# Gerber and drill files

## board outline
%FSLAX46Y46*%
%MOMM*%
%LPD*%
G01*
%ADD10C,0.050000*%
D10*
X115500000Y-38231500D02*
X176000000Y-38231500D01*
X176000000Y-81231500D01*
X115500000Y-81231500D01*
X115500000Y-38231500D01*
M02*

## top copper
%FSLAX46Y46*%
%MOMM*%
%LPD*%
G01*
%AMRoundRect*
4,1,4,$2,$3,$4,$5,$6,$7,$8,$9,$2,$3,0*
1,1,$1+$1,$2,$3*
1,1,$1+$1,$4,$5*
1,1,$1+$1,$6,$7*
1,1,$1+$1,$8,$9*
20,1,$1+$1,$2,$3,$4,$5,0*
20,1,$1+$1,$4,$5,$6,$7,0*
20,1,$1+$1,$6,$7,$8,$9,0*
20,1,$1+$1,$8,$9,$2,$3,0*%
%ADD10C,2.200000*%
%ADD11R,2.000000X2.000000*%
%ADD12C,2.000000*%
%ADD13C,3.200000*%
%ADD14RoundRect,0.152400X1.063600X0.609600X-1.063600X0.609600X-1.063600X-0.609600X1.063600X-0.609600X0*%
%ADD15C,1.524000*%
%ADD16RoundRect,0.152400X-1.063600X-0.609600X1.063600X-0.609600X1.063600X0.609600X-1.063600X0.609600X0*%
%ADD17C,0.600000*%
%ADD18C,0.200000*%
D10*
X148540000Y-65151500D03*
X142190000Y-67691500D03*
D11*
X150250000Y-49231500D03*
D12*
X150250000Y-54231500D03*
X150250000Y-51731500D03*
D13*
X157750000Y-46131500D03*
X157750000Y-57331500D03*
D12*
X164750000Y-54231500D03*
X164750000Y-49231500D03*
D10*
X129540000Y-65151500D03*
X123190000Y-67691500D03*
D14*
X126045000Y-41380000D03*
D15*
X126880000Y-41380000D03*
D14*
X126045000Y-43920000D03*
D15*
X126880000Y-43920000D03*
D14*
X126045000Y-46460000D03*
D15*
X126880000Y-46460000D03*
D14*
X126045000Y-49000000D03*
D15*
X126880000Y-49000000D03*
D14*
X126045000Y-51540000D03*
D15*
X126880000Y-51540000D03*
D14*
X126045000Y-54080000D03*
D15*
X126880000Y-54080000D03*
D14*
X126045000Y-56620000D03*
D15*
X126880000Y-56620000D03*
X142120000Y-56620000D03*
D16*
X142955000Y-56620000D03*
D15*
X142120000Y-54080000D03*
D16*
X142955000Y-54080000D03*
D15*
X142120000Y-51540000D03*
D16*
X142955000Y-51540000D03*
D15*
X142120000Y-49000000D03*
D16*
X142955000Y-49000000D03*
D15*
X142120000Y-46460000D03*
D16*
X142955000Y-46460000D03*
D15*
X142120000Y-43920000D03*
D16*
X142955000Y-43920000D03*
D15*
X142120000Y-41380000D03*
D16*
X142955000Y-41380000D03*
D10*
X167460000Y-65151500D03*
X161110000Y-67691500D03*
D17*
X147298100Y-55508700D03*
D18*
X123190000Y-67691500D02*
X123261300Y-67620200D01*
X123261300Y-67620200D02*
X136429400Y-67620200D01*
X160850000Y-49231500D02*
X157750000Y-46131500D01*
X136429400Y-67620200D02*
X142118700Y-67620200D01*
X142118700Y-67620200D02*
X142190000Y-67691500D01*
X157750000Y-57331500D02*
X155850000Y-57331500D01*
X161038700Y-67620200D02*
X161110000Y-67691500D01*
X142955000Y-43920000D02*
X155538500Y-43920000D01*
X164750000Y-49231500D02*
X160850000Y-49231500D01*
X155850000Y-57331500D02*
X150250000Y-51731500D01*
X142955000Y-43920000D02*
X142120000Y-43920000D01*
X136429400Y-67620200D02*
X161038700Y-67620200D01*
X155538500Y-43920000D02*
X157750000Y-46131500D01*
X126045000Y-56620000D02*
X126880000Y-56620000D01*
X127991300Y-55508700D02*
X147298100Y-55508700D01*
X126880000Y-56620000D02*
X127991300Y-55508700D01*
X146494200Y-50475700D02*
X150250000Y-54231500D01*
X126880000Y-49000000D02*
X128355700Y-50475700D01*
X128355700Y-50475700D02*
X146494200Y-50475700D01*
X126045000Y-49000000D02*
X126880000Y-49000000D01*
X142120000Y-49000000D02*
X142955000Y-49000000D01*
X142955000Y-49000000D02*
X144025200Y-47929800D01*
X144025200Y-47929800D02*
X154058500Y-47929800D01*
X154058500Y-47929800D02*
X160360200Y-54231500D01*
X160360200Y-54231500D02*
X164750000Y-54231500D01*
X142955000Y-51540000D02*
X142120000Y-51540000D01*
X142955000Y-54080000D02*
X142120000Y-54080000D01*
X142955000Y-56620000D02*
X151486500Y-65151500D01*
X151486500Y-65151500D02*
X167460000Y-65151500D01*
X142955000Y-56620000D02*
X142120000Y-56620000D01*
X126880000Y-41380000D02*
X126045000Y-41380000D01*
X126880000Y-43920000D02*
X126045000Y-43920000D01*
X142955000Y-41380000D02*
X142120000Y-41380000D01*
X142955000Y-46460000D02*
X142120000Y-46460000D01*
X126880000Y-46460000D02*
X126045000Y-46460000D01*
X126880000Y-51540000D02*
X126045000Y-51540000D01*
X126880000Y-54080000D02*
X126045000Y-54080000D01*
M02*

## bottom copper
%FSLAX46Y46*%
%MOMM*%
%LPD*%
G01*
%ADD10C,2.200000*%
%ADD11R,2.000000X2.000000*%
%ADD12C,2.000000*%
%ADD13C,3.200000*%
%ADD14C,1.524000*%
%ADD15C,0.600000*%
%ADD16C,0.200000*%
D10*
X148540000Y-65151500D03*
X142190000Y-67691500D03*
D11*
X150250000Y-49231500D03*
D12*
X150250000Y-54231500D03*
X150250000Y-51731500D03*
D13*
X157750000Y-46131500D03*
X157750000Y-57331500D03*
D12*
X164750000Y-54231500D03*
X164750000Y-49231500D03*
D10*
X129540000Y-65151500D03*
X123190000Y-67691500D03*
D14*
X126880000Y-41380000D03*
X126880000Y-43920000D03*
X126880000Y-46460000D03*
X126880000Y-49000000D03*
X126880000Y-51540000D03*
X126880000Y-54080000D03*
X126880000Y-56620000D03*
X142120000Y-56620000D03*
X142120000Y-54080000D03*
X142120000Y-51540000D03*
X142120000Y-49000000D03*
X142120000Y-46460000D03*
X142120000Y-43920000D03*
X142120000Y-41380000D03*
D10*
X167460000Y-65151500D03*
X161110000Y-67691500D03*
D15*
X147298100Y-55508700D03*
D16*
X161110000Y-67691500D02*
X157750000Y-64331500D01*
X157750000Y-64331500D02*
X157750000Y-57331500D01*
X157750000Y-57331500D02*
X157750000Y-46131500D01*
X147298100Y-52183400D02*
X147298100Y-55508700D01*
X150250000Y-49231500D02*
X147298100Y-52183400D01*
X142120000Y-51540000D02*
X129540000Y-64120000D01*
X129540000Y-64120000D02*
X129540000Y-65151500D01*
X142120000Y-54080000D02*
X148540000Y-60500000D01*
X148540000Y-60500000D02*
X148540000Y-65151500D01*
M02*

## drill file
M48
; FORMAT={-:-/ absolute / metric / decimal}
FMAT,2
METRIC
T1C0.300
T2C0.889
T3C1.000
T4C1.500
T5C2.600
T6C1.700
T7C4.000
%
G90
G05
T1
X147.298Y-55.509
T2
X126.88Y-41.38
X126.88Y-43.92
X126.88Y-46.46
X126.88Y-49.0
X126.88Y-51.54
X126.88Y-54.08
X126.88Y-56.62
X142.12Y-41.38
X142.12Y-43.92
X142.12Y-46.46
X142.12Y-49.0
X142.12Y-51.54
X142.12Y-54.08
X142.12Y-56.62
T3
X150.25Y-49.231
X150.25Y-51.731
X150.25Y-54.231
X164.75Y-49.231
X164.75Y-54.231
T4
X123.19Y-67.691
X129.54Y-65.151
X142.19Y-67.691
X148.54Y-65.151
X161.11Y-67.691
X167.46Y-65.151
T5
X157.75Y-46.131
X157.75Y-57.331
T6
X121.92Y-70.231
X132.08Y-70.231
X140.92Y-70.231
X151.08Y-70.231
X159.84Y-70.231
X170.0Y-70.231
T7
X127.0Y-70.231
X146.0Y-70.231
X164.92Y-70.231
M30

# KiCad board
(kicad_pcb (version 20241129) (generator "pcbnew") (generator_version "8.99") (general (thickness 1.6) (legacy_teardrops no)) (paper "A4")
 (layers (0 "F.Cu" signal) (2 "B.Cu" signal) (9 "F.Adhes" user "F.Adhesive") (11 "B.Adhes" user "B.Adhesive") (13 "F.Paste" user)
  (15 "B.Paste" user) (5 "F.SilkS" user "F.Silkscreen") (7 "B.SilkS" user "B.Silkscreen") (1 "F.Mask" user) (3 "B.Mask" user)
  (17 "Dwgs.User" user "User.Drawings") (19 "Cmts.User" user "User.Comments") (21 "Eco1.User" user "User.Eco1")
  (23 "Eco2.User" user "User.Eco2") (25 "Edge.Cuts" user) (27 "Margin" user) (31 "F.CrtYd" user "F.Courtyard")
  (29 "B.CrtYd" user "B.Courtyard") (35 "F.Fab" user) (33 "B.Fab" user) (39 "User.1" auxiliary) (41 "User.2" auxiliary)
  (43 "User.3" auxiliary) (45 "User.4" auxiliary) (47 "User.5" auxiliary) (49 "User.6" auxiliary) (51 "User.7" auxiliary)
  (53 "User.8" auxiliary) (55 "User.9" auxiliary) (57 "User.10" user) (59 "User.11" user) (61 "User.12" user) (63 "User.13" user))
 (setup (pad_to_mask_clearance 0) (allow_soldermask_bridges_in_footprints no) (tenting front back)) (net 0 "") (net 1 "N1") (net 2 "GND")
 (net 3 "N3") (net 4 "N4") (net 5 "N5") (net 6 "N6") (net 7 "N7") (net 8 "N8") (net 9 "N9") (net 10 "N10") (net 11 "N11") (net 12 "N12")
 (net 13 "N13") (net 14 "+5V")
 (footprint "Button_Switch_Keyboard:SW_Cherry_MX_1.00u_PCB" (layer "F.Cu") (at 148.54 65.1515)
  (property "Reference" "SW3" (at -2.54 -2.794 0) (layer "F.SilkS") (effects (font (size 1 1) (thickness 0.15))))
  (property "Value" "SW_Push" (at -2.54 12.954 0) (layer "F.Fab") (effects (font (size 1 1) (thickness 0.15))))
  (pad "" np_thru_hole circle (at -7.62 5.08) (size 1.7 1.7) (drill 1.7) (layers "*.Cu" "*.Mask"))
  (pad "" np_thru_hole circle (at -2.54 5.08) (size 4 4) (drill 4) (layers "*.Cu" "*.Mask"))
  (pad "" np_thru_hole circle (at 2.54 5.08) (size 1.7 1.7) (drill 1.7) (layers "*.Cu" "*.Mask"))
  (pad "1" thru_hole circle (at 0 0) (size 2.2 2.2) (drill 1.5) (layers "*.Cu" "*.Mask") (remove_unused_layers no) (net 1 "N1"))
  (pad "2" thru_hole circle (at -6.35 2.54) (size 2.2 2.2) (drill 1.5) (layers "*.Cu" "*.Mask") (remove_unused_layers no) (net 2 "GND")))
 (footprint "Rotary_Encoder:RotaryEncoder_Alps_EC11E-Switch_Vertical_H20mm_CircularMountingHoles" (layer "F.Cu") (at 150.25 49.2315)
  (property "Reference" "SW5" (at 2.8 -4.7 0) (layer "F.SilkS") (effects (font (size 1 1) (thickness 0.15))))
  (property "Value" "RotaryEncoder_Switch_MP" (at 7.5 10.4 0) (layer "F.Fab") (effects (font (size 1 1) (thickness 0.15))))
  (pad "A" thru_hole rect (at 0 0) (size 2 2) (drill 1) (layers "*.Cu" "*.Mask") (remove_unused_layers no) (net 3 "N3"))
  (pad "B" thru_hole circle (at 0 5) (size 2 2) (drill 1) (layers "*.Cu" "*.Mask") (remove_unused_layers no) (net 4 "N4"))
  (pad "C" thru_hole circle (at 0 2.5) (size 2 2) (drill 1) (layers "*.Cu" "*.Mask") (remove_unused_layers no) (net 2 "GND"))
  (pad "MP" thru_hole circle (at 7.5 -3.1) (size 3.2 3.2) (drill 2.6) (layers "*.Cu" "*.Mask") (remove_unused_layers no) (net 2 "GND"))
  (pad "MP" thru_hole circle (at 7.5 8.1) (size 3.2 3.2) (drill 2.6) (layers "*.Cu" "*.Mask") (remove_unused_layers no) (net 2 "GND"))
  (pad "S1" thru_hole circle (at 14.5 5) (size 2 2) (drill 1) (layers "*.Cu" "*.Mask") (remove_unused_layers no) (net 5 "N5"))
  (pad "S2" thru_hole circle (at 14.5 0) (size 2 2) (drill 1) (layers "*.Cu" "*.Mask") (remove_unused_layers no) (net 2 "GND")))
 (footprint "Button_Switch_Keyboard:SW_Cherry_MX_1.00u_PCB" (layer "F.Cu") (at 129.54 65.1515)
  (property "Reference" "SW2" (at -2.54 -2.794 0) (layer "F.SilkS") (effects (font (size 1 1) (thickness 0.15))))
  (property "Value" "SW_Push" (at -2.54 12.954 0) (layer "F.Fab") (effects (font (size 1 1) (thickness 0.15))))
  (pad "" np_thru_hole circle (at -7.62 5.08) (size 1.7 1.7) (drill 1.7) (layers "*.Cu" "*.Mask"))
  (pad "" np_thru_hole circle (at -2.54 5.08) (size 4 4) (drill 4) (layers "*.Cu" "*.Mask"))
  (pad "" np_thru_hole circle (at 2.54 5.08) (size 1.7 1.7) (drill 1.7) (layers "*.Cu" "*.Mask"))
  (pad "1" thru_hole circle (at 0 0) (size 2.2 2.2) (drill 1.5) (layers "*.Cu" "*.Mask") (remove_unused_layers no) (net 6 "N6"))
  (pad "2" thru_hole circle (at -6.35 2.54) (size 2.2 2.2) (drill 1.5) (layers "*.Cu" "*.Mask") (remove_unused_layers no) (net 2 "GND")))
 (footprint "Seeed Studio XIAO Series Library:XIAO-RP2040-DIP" (layer "F.Cu") (at 134.5 49)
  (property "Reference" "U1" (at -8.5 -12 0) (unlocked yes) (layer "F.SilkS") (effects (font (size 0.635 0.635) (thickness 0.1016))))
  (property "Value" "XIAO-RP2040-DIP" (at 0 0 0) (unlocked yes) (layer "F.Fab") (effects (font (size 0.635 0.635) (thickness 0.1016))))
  (pad "1" smd roundrect (at -8.455 -7.62 180) (size 2.432 1.524) (layers "F.Cu" "F.Mask") (roundrect_rratio 0.1) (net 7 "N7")
   (thermal_bridge_angle 45))
  (pad "1" thru_hole circle (at -7.62 -7.62 180) (size 1.524 1.524) (drill 0.889) (layers "*.Cu" "*.Mask") (remove_unused_layers no)
   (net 7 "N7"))
  (pad "2" smd roundrect (at -8.455 -5.08 180) (size 2.432 1.524) (layers "F.Cu" "F.Mask") (roundrect_rratio 0.1) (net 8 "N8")
   (thermal_bridge_angle 45))
  (pad "2" thru_hole circle (at -7.62 -5.08 180) (size 1.524 1.524) (drill 0.889) (layers "*.Cu" "*.Mask") (remove_unused_layers no)
   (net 8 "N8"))
  (pad "3" smd roundrect (at -8.455 -2.54 180) (size 2.432 1.524) (layers "F.Cu" "F.Mask") (roundrect_rratio 0.1) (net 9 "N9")
   (thermal_bridge_angle 45))
  (pad "3" thru_hole circle (at -7.62 -2.54 180) (size 1.524 1.524) (drill 0.889) (layers "*.Cu" "*.Mask") (remove_unused_layers no)
   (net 9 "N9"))
  (pad "4" smd roundrect (at -8.455 0 180) (size 2.432 1.524) (layers "F.Cu" "F.Mask") (roundrect_rratio 0.1) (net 4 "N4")
   (thermal_bridge_angle 45))
  (pad "4" thru_hole circle (at -7.62 0 180) (size 1.524 1.524) (drill 0.889) (layers "*.Cu" "*.Mask") (remove_unused_layers no)
   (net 4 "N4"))
  (pad "5" smd roundrect (at -8.455 2.54 180) (size 2.432 1.524) (layers "F.Cu" "F.Mask") (roundrect_rratio 0.1) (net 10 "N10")
   (thermal_bridge_angle 45))
  (pad "5" thru_hole circle (at -7.62 2.54 180) (size 1.524 1.524) (drill 0.889) (layers "*.Cu" "*.Mask") (remove_unused_layers no)
   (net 10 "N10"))
  (pad "6" smd roundrect (at -8.455 5.08 180) (size 2.432 1.524) (layers "F.Cu" "F.Mask") (roundrect_rratio 0.1) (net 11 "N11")
   (thermal_bridge_angle 45))
  (pad "6" thru_hole circle (at -7.62 5.08 180) (size 1.524 1.524) (drill 0.889) (layers "*.Cu" "*.Mask") (remove_unused_layers no)
   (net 11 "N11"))
  (pad "7" smd roundrect (at -8.455 7.62 180) (size 2.432 1.524) (layers "F.Cu" "F.Mask") (roundrect_rratio 0.1) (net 3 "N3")
   (thermal_bridge_angle 45))
  (pad "7" thru_hole circle (at -7.62 7.62 180) (size 1.524 1.524) (drill 0.889) (layers "*.Cu" "*.Mask") (remove_unused_layers no)
   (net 3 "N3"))
  (pad "8" thru_hole circle (at 7.62 7.62) (size 1.524 1.524) (drill 0.889) (layers "*.Cu" "*.Mask") (remove_unused_layers no)
   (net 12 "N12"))
  (pad "8" smd roundrect (at 8.455 7.62) (size 2.432 1.524) (layers "F.Cu" "F.Mask") (roundrect_rratio 0.1) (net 12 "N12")
   (thermal_bridge_angle 45))
  (pad "9" thru_hole circle (at 7.62 5.08) (size 1.524 1.524) (drill 0.889) (layers "*.Cu" "*.Mask") (remove_unused_layers no) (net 1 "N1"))
  (pad "9" smd roundrect (at 8.455 5.08) (size 2.432 1.524) (layers "F.Cu" "F.Mask") (roundrect_rratio 0.1) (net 1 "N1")
   (thermal_bridge_angle 45))
  (pad "10" thru_hole circle (at 7.62 2.54) (size 1.524 1.524) (drill 0.889) (layers "*.Cu" "*.Mask") (remove_unused_layers no) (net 6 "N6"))
  (pad "10" smd roundrect (at 8.455 2.54) (size 2.432 1.524) (layers "F.Cu" "F.Mask") (roundrect_rratio 0.1) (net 6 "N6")
   (thermal_bridge_angle 45))
  (pad "11" thru_hole circle (at 7.62 0) (size 1.524 1.524) (drill 0.889) (layers "*.Cu" "*.Mask") (remove_unused_layers no) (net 5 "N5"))
  (pad "11" smd roundrect (at 8.455 0) (size 2.432 1.524) (layers "F.Cu" "F.Mask") (roundrect_rratio 0.1) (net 5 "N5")
   (thermal_bridge_angle 45))
  (pad "12" thru_hole circle (at 7.62 -2.54) (size 1.524 1.524) (drill 0.889) (layers "*.Cu" "*.Mask") (remove_unused_layers no)
   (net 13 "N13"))
  (pad "12" smd roundrect (at 8.455 -2.54) (size 2.432 1.524) (layers "F.Cu" "F.Mask") (roundrect_rratio 0.1) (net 13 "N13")
   (thermal_bridge_angle 45))
  (pad "13" thru_hole circle (at 7.62 -5.08) (size 1.524 1.524) (drill 0.889) (layers "*.Cu" "*.Mask") (remove_unused_layers no)
   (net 2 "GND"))
  (pad "13" smd roundrect (at 8.455 -5.08) (size 2.432 1.524) (layers "F.Cu" "F.Mask") (roundrect_rratio 0.1) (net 2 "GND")
   (thermal_bridge_angle 45))
  (pad "14" thru_hole circle (at 7.62 -7.62) (size 1.524 1.524) (drill 0.889) (layers "*.Cu" "*.Mask") (remove_unused_layers no)
   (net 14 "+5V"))
  (pad "14" smd roundrect (at 8.455 -7.62) (size 2.432 1.524) (layers "F.Cu" "F.Mask") (roundrect_rratio 0.1) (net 14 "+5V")
   (thermal_bridge_angle 45)))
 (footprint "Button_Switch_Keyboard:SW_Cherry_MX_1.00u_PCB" (layer "F.Cu") (at 167.46 65.1515)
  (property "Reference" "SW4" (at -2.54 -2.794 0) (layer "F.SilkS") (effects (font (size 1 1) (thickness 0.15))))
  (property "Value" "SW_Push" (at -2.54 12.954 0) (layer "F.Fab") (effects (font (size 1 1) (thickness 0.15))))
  (pad "" np_thru_hole circle (at -7.62 5.08) (size 1.7 1.7) (drill 1.7) (layers "*.Cu" "*.Mask"))
  (pad "" np_thru_hole circle (at -2.54 5.08) (size 4 4) (drill 4) (layers "*.Cu" "*.Mask"))
  (pad "" np_thru_hole circle (at 2.54 5.08) (size 1.7 1.7) (drill 1.7) (layers "*.Cu" "*.Mask"))
  (pad "1" thru_hole circle (at 0 0) (size 2.2 2.2) (drill 1.5) (layers "*.Cu" "*.Mask") (remove_unused_layers no) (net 12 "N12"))
  (pad "2" thru_hole circle (at -6.35 2.54) (size 2.2 2.2) (drill 1.5) (layers "*.Cu" "*.Mask") (remove_unused_layers no) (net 2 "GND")))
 (gr_rect (start 115.5 38.2315) (end 176 81.2315) (stroke (width 0.05) (type default)) (fill no) (layer "Edge.Cuts"))
 (segment (start 123.19 67.6915) (end 123.2613 67.6202) (width 0.2) (layer "F.Cu") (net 2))
 (segment (start 123.2613 67.6202) (end 136.4294 67.6202) (width 0.2) (layer "F.Cu") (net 2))
 (segment (start 160.85 49.2315) (end 157.75 46.1315) (width 0.2) (layer "F.Cu") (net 2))
 (segment (start 136.4294 67.6202) (end 142.1187 67.6202) (width 0.2) (layer "F.Cu") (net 2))
 (segment (start 142.1187 67.6202) (end 142.19 67.6915) (width 0.2) (layer "F.Cu") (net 2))
 (segment (start 157.75 57.3315) (end 155.85 57.3315) (width 0.2) (layer "F.Cu") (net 2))
 (segment (start 161.0387 67.6202) (end 161.11 67.6915) (width 0.2) (layer "F.Cu") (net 2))
 (segment (start 142.955 43.92) (end 155.5385 43.92) (width 0.2) (layer "F.Cu") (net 2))
 (segment (start 164.75 49.2315) (end 160.85 49.2315) (width 0.2) (layer "F.Cu") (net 2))
 (segment (start 155.85 57.3315) (end 150.25 51.7315) (width 0.2) (layer "F.Cu") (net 2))
 (segment (start 142.955 43.92) (end 142.12 43.92) (width 0.2) (layer "F.Cu") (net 2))
 (segment (start 136.4294 67.6202) (end 161.0387 67.6202) (width 0.2) (layer "F.Cu") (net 2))
 (segment (start 155.5385 43.92) (end 157.75 46.1315) (width 0.2) (layer "F.Cu") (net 2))
 (segment (start 161.11 67.6915) (end 157.75 64.3315) (width 0.2) (layer "B.Cu") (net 2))
 (segment (start 157.75 64.3315) (end 157.75 57.3315) (width 0.2) (layer "B.Cu") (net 2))
 (segment (start 157.75 57.3315) (end 157.75 46.1315) (width 0.2) (layer "B.Cu") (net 2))
 (segment (start 126.045 56.62) (end 126.88 56.62) (width 0.2) (layer "F.Cu") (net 3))
 (segment (start 127.9913 55.5087) (end 147.2981 55.5087) (width 0.2) (layer "F.Cu") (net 3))
 (segment (start 126.88 56.62) (end 127.9913 55.5087) (width 0.2) (layer "F.Cu") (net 3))
 (via (at 147.2981 55.5087) (size 0.6) (drill 0.3) (layers "F.Cu" "B.Cu") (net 3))
 (segment (start 147.2981 52.1834) (end 147.2981 55.5087) (width 0.2) (layer "B.Cu") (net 3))
 (segment (start 150.25 49.2315) (end 147.2981 52.1834) (width 0.2) (layer "B.Cu") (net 3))
 (segment (start 146.4942 50.4757) (end 150.25 54.2315) (width 0.2) (layer "F.Cu") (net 4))
 (segment (start 126.88 49) (end 128.3557 50.4757) (width 0.2) (layer "F.Cu") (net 4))
 (segment (start 128.3557 50.4757) (end 146.4942 50.4757) (width 0.2) (layer "F.Cu") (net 4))
 (segment (start 126.045 49) (end 126.88 49) (width 0.2) (layer "F.Cu") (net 4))
 (segment (start 142.12 49) (end 142.955 49) (width 0.2) (layer "F.Cu") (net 5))
 (segment (start 142.955 49) (end 144.0252 47.9298) (width 0.2) (layer "F.Cu") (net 5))
 (segment (start 144.0252 47.9298) (end 154.0585 47.9298) (width 0.2) (layer "F.Cu") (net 5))
 (segment (start 154.0585 47.9298) (end 160.3602 54.2315) (width 0.2) (layer "F.Cu") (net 5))
 (segment (start 160.3602 54.2315) (end 164.75 54.2315) (width 0.2) (layer "F.Cu") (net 5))
 (segment (start 142.955 51.54) (end 142.12 51.54) (width 0.2) (layer "F.Cu") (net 6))
 (segment (start 142.12 51.54) (end 129.54 64.12) (width 0.2) (layer "B.Cu") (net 6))
 (segment (start 129.54 64.12) (end 129.54 65.1515) (width 0.2) (layer "B.Cu") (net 6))
 (segment (start 142.955 54.08) (end 142.12 54.08) (width 0.2) (layer "F.Cu") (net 1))
 (segment (start 142.12 54.08) (end 148.54 60.5) (width 0.2) (layer "B.Cu") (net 1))
 (segment (start 148.54 60.5) (end 148.54 65.1515) (width 0.2) (layer "B.Cu") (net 1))
 (segment (start 142.955 56.62) (end 151.4865 65.1515) (width 0.2) (layer "F.Cu") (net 12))
 (segment (start 151.4865 65.1515) (end 167.46 65.1515) (width 0.2) (layer "F.Cu") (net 12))
 (segment (start 142.955 56.62) (end 142.12 56.62) (width 0.2) (layer "F.Cu") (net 12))
 (segment (start 126.88 41.38) (end 126.045 41.38) (width 0.2) (layer "F.Cu") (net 7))
 (segment (start 126.88 43.92) (end 126.045 43.92) (width 0.2) (layer "F.Cu") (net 8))
 (segment (start 142.955 41.38) (end 142.12 41.38) (width 0.2) (layer "F.Cu") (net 14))
 (segment (start 142.955 46.46) (end 142.12 46.46) (width 0.2) (layer "F.Cu") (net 13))
 (segment (start 126.88 46.46) (end 126.045 46.46) (width 0.2) (layer "F.Cu") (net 9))
 (segment (start 126.88 51.54) (end 126.045 51.54) (width 0.2) (layer "F.Cu") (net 10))
 (segment (start 126.88 54.08) (end 126.045 54.08) (width 0.2) (layer "F.Cu") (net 11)))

